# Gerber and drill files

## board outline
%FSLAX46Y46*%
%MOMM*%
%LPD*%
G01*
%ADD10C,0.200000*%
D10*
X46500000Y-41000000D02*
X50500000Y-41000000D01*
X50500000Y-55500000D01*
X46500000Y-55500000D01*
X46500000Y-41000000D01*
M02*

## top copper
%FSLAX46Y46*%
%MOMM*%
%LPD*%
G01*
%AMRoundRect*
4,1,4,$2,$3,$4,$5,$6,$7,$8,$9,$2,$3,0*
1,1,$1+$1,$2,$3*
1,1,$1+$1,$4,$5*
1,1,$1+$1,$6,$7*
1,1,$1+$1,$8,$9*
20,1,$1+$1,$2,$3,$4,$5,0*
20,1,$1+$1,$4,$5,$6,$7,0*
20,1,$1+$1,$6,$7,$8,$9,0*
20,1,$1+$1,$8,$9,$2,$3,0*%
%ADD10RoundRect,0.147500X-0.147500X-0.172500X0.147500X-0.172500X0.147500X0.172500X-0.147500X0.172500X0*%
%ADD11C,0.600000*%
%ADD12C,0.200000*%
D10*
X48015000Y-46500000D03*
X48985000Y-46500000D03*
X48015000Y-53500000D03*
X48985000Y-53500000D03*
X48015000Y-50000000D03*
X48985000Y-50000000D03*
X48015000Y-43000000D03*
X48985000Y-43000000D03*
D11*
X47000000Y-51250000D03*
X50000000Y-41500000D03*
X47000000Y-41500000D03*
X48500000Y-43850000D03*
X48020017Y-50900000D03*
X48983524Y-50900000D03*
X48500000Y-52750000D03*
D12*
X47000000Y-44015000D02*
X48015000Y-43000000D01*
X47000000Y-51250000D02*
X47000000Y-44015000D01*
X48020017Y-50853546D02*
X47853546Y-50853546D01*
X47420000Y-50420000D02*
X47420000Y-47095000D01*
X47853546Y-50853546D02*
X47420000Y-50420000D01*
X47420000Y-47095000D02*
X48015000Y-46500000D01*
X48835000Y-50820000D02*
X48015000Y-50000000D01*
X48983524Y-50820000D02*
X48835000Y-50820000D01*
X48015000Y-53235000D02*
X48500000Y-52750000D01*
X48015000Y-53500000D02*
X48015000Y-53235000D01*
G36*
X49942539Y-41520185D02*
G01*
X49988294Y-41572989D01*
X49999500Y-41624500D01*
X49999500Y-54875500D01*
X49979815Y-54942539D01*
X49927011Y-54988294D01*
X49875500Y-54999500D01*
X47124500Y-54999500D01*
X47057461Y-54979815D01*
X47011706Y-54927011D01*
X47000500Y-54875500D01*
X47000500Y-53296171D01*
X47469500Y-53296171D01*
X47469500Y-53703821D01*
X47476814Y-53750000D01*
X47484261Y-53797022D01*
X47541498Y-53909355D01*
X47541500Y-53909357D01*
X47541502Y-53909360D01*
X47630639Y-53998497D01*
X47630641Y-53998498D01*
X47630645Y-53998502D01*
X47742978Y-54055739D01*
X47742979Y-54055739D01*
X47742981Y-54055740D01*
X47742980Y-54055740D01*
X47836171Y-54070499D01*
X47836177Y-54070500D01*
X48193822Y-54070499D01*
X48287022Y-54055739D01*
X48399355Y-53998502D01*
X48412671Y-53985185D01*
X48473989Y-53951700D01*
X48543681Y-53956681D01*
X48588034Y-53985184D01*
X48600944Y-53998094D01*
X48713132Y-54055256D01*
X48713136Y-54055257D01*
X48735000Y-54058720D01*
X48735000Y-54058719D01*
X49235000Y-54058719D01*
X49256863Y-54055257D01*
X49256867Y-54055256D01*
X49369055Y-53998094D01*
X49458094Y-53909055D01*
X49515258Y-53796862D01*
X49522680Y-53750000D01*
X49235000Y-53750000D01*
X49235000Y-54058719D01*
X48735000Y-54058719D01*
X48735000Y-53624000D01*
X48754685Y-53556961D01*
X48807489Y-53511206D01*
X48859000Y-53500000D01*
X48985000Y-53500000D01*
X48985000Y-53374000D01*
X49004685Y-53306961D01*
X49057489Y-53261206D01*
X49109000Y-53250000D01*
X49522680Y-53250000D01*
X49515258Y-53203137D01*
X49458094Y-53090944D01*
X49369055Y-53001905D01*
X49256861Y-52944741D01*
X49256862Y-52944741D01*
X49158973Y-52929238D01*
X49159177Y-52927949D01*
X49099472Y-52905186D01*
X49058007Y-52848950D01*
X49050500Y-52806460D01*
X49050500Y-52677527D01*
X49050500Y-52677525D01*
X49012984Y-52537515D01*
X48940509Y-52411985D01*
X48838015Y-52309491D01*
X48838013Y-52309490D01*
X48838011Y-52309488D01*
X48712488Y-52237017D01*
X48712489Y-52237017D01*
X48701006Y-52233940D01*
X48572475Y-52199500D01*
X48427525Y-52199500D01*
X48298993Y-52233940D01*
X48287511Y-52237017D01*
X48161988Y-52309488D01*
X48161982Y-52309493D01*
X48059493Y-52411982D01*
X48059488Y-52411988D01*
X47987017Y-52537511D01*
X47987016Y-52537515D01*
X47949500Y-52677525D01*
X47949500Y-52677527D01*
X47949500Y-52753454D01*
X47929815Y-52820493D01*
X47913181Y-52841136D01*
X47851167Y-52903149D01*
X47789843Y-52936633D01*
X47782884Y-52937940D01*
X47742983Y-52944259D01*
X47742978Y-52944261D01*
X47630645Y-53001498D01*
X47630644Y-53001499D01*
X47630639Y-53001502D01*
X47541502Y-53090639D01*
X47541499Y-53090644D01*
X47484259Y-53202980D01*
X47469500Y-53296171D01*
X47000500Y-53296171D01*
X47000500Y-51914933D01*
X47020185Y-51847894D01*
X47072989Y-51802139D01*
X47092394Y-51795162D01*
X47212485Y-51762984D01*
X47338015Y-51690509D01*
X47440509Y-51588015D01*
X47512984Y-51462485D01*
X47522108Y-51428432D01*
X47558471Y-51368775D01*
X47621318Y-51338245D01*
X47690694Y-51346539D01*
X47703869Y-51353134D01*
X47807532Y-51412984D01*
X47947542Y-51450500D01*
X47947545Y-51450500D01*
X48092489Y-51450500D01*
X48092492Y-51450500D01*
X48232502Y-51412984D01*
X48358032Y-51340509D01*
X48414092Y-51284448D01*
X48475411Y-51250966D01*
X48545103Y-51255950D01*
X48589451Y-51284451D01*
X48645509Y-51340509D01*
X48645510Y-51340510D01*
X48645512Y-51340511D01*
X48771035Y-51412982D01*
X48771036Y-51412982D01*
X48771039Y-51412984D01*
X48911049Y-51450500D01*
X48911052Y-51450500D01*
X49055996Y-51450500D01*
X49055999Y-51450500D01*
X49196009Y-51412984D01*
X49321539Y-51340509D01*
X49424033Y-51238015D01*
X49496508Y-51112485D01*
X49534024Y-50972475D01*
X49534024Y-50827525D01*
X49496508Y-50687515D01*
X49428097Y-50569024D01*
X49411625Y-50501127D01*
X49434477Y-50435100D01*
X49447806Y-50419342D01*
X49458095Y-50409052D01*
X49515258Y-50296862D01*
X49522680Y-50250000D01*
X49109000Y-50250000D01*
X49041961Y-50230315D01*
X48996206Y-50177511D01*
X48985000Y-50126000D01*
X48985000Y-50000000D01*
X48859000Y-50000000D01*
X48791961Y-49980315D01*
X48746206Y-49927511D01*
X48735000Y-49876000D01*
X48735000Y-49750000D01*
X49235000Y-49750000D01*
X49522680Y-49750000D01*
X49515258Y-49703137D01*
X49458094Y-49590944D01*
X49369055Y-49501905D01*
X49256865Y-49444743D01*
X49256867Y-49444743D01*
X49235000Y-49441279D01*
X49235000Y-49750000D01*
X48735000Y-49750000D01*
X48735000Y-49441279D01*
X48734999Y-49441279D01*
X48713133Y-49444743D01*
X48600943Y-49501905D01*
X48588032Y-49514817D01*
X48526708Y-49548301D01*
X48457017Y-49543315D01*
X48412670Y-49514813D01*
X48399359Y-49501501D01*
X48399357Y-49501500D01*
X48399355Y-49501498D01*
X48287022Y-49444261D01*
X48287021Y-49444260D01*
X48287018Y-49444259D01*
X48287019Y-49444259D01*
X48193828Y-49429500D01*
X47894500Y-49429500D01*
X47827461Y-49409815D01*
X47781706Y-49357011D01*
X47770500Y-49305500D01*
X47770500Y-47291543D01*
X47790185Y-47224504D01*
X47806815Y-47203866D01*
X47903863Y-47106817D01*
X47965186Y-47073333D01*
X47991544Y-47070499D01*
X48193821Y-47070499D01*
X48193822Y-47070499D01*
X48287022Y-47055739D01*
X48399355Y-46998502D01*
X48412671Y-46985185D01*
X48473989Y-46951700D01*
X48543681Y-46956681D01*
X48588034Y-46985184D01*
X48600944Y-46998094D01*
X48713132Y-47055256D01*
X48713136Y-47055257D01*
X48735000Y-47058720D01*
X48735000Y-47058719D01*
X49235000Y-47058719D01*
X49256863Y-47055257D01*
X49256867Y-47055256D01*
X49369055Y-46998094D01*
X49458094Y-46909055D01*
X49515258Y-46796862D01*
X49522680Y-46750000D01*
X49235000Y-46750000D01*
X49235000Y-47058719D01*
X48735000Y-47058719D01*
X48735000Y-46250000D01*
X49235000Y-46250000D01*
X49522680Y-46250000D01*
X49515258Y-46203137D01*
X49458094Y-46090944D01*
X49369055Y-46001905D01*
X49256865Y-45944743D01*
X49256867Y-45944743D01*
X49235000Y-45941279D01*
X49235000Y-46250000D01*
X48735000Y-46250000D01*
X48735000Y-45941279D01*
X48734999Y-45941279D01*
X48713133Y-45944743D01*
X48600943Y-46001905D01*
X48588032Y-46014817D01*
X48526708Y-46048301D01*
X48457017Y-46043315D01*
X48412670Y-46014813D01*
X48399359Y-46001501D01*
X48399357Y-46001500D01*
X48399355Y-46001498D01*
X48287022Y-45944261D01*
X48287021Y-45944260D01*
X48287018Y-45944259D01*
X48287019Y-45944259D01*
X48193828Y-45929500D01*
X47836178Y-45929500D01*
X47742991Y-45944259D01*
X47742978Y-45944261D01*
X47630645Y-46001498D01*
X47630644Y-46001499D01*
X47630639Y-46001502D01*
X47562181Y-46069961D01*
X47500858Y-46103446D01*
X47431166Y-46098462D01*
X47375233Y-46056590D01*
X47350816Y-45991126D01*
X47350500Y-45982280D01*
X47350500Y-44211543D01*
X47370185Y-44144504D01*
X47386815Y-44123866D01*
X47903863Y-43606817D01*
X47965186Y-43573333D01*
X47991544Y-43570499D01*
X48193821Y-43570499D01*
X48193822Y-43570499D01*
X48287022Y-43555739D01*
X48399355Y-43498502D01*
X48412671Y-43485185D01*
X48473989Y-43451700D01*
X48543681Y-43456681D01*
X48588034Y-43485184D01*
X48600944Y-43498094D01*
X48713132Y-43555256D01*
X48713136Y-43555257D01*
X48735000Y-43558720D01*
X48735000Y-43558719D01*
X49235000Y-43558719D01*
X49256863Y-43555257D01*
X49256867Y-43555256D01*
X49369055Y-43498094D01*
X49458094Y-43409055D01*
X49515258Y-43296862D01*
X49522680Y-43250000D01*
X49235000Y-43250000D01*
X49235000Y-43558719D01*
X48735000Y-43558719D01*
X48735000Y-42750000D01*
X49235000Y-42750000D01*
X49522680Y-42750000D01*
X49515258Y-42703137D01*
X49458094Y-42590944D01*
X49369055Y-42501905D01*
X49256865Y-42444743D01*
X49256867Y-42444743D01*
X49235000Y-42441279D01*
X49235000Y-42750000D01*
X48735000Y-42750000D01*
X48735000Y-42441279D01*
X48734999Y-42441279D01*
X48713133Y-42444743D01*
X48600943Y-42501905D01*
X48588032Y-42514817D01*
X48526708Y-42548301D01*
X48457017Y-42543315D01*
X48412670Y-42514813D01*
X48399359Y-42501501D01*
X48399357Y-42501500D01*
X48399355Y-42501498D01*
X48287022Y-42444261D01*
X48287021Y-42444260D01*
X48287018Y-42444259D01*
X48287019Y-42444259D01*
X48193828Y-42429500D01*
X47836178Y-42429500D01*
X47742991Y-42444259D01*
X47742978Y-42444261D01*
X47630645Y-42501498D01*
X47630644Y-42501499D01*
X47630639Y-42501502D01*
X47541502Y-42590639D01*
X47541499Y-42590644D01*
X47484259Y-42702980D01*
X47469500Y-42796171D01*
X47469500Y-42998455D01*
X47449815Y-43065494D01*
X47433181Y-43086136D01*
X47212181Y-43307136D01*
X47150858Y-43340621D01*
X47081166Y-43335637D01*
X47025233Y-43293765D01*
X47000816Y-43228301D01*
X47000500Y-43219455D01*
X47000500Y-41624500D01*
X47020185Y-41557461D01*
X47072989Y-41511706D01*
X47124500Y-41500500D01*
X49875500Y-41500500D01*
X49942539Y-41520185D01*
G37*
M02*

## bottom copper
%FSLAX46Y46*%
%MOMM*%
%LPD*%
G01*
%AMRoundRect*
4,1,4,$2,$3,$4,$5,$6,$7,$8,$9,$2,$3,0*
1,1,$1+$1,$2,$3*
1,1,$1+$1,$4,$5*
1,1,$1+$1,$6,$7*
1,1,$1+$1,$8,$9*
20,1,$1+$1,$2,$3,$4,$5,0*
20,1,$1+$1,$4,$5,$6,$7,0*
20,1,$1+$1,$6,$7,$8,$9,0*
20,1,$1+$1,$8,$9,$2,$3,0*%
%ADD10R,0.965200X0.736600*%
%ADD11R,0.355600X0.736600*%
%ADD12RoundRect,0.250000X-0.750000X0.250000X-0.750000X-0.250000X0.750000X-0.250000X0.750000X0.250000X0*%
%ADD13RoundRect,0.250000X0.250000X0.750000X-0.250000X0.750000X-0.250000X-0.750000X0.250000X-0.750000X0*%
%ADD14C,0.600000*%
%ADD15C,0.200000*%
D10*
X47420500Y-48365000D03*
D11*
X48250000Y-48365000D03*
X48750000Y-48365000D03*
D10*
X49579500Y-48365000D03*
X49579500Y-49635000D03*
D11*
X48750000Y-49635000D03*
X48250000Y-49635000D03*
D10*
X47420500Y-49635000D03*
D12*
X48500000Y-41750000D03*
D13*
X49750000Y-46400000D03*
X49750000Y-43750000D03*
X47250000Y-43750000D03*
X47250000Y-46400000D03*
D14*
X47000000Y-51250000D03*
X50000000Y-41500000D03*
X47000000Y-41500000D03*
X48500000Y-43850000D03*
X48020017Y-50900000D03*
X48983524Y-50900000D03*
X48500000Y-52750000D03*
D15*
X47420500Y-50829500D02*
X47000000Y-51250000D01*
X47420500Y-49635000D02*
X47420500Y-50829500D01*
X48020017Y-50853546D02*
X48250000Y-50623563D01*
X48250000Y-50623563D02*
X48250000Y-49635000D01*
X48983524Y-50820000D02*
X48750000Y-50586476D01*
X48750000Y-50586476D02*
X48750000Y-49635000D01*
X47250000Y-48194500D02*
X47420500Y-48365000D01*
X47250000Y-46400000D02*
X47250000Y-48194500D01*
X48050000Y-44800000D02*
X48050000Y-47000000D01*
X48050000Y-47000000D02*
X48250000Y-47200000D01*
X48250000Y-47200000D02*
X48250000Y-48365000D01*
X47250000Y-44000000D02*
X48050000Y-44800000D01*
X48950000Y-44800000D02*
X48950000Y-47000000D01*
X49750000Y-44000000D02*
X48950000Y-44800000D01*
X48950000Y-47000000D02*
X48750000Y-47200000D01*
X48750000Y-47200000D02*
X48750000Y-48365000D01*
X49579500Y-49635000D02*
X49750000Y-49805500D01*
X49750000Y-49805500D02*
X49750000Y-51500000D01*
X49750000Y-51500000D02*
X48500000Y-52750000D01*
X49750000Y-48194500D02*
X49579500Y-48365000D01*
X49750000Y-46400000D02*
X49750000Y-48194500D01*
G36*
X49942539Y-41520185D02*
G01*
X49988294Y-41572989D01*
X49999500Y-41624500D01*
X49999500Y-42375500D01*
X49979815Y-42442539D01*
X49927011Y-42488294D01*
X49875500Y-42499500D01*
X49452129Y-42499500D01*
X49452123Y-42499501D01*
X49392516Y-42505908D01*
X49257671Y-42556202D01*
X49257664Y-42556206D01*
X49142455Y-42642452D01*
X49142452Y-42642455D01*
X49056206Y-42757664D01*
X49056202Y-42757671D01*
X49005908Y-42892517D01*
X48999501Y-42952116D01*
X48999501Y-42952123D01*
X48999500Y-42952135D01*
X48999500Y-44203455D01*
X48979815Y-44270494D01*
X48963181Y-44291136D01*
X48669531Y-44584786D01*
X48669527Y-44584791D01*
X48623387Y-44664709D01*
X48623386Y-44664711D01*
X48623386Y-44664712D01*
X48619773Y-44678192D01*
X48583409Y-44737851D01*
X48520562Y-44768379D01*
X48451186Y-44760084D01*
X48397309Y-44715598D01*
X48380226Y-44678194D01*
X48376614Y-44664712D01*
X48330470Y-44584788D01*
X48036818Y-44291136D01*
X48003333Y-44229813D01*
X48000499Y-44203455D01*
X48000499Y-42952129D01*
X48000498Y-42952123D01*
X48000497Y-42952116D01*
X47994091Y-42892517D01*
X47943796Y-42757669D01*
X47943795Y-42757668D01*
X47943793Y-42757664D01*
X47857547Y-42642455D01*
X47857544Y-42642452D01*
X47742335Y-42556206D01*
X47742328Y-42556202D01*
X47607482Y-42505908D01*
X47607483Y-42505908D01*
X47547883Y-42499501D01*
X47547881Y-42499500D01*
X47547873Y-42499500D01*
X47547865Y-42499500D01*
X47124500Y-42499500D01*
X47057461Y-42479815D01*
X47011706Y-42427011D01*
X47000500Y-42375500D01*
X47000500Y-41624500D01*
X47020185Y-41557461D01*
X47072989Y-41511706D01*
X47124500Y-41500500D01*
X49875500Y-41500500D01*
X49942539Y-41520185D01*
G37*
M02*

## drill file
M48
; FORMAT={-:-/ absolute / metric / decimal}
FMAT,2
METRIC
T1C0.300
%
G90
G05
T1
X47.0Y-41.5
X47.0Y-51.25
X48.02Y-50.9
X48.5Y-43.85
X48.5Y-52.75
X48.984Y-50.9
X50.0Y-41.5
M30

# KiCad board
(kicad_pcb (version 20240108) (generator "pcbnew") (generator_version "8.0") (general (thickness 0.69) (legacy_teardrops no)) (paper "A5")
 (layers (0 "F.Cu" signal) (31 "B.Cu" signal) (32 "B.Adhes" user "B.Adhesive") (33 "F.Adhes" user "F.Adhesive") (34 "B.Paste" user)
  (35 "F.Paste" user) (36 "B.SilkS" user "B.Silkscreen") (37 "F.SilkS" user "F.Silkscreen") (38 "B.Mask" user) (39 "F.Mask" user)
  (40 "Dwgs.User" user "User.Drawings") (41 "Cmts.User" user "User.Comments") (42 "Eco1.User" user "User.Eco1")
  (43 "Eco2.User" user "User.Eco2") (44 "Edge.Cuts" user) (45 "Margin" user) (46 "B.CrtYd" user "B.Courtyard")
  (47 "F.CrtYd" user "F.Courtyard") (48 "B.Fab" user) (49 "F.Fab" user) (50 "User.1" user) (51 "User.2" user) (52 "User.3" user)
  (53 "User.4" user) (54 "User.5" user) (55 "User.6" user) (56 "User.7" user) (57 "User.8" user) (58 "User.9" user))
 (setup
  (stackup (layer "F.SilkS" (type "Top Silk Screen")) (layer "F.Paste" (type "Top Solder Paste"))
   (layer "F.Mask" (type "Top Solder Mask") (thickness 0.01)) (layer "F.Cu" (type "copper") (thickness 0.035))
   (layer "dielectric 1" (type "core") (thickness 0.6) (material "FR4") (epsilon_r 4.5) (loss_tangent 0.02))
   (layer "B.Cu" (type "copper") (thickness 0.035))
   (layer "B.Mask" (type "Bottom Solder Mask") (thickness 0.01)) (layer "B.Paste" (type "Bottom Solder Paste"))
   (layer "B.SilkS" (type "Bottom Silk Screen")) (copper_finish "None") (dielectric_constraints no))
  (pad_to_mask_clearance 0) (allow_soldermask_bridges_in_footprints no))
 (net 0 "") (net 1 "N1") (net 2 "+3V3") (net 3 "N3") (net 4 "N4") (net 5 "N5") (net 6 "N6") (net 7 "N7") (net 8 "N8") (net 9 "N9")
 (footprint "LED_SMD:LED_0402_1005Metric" (layer "F.Cu") (at 48.5 46.5)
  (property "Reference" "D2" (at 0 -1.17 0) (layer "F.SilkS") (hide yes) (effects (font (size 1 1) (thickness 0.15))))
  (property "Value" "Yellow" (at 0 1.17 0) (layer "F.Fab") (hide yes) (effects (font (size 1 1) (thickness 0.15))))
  (pad "1" smd roundrect (at -0.485 0) (size 0.59 0.64) (layers "F.Cu" "F.Paste" "F.Mask") (roundrect_rratio 0.25) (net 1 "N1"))
  (pad "2" smd roundrect (at 0.485 0) (size 0.59 0.64) (layers "F.Cu" "F.Paste" "F.Mask") (roundrect_rratio 0.25) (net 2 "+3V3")))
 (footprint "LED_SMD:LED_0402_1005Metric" (layer "F.Cu") (at 48.5 53.5)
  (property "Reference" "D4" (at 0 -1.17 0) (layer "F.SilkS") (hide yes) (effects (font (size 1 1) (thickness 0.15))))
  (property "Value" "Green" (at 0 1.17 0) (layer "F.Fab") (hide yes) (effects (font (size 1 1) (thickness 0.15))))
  (pad "1" smd roundrect (at -0.485 0) (size 0.59 0.64) (layers "F.Cu" "F.Paste" "F.Mask") (roundrect_rratio 0.25) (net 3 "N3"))
  (pad "2" smd roundrect (at 0.485 0) (size 0.59 0.64) (layers "F.Cu" "F.Paste" "F.Mask") (roundrect_rratio 0.25) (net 2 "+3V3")))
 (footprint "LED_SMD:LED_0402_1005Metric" (layer "F.Cu") (at 48.5 50)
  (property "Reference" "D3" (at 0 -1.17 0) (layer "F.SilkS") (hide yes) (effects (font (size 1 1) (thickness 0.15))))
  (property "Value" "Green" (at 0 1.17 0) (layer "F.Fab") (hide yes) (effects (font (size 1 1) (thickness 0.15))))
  (pad "1" smd roundrect (at -0.485 0) (size 0.59 0.64) (layers "F.Cu" "F.Paste" "F.Mask") (roundrect_rratio 0.25) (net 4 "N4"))
  (pad "2" smd roundrect (at 0.485 0) (size 0.59 0.64) (layers "F.Cu" "F.Paste" "F.Mask") (roundrect_rratio 0.25) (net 2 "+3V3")))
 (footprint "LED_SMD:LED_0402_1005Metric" (layer "F.Cu") (at 48.5 43)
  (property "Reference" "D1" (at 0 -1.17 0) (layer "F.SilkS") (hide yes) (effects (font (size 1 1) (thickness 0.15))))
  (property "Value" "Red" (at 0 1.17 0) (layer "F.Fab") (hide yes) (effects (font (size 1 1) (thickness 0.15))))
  (pad "1" smd roundrect (at -0.485 0) (size 0.59 0.64) (layers "F.Cu" "F.Paste" "F.Mask") (roundrect_rratio 0.25) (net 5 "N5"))
  (pad "2" smd roundrect (at 0.485 0) (size 0.59 0.64) (layers "F.Cu" "F.Paste" "F.Mask") (roundrect_rratio 0.25) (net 2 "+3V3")))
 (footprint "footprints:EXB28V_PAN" (layer "B.Cu") (at 48.5 49 -90)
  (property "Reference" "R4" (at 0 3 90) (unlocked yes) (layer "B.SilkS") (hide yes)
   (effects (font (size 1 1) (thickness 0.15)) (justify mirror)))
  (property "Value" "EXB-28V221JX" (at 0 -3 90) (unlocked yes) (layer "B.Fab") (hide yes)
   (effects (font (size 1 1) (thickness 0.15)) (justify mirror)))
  (pad "1" smd rect (at -0.635 1.0795 270) (size 0.7366 0.9652) (layers "B.Cu" "B.Paste" "B.Mask") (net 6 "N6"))
  (pad "2" smd rect (at -0.635 0.25 270) (size 0.7366 0.3556) (layers "B.Cu" "B.Paste" "B.Mask") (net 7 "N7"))
  (pad "3" smd rect (at -0.635 -0.25 270) (size 0.7366 0.3556) (layers "B.Cu" "B.Paste" "B.Mask") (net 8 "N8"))
  (pad "4" smd rect (at -0.635 -1.0795 270) (size 0.7366 0.9652) (layers "B.Cu" "B.Paste" "B.Mask") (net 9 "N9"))
  (pad "5" smd rect (at 0.635 -1.0795 270) (size 0.7366 0.9652) (layers "B.Cu" "B.Paste" "B.Mask") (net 3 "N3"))
  (pad "6" smd rect (at 0.635 -0.25 270) (size 0.7366 0.3556) (layers "B.Cu" "B.Paste" "B.Mask") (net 4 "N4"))
  (pad "7" smd rect (at 0.635 0.25 270) (size 0.7366 0.3556) (layers "B.Cu" "B.Paste" "B.Mask") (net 1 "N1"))
  (pad "8" smd rect (at 0.635 1.0795 270) (size 0.7366 0.9652) (layers "B.Cu" "B.Paste" "B.Mask") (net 5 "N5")))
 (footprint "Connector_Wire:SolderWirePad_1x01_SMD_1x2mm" (layer "B.Cu") (at 48.5 41.75 -90)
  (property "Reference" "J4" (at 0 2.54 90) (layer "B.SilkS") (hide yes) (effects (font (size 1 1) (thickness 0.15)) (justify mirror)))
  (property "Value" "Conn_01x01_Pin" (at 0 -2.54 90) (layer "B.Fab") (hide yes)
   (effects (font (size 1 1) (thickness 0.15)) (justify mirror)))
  (pad "1" smd roundrect (at 0 0 270) (size 1 2) (layers "B.Cu" "B.Paste" "B.Mask") (roundrect_rratio 0.25) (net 2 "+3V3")))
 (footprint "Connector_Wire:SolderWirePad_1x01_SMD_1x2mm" (layer "B.Cu") (at 49.75 46.4 180)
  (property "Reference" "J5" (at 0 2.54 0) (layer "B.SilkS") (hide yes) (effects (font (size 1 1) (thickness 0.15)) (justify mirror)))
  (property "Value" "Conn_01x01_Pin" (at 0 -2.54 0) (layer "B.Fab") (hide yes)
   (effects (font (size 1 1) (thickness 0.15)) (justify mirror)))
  (pad "1" smd roundrect (at 0 0 180) (size 1 2) (layers "B.Cu" "B.Paste" "B.Mask") (roundrect_rratio 0.25) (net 9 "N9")))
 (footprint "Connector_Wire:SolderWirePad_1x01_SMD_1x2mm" (layer "B.Cu") (at 49.75 43.75 180)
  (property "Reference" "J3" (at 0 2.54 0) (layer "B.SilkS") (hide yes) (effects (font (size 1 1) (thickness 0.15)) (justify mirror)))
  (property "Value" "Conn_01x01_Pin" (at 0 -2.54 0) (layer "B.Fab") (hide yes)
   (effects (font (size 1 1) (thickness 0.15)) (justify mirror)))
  (pad "1" smd roundrect (at 0 0 180) (size 1 2) (layers "B.Cu" "B.Paste" "B.Mask") (roundrect_rratio 0.25) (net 8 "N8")))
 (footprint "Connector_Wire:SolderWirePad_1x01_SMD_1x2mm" (layer "B.Cu") (at 47.25 43.75 180)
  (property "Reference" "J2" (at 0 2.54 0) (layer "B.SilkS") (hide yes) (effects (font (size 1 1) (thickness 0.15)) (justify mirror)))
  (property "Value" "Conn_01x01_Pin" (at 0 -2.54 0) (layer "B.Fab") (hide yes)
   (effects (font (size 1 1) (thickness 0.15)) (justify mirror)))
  (pad "1" smd roundrect (at 0 0 180) (size 1 2) (layers "B.Cu" "B.Paste" "B.Mask") (roundrect_rratio 0.25) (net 7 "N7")))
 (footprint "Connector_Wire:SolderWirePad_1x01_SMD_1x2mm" (layer "B.Cu") (at 47.25 46.4 180)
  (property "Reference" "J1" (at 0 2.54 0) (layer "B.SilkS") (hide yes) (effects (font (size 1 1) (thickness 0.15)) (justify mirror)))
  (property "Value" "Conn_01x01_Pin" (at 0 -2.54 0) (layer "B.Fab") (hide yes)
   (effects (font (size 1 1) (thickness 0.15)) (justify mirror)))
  (pad "1" smd roundrect (at 0 0 180) (size 1 2) (layers "B.Cu" "B.Paste" "B.Mask") (roundrect_rratio 0.25) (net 6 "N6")))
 (gr_rect (start 46.5 41) (end 50.5 55.5) (stroke (width 0.2) (type default)) (fill none) (layer "Edge.Cuts"))
 (segment (start 47 44.015) (end 48.015 43) (width 0.2) (layer "F.Cu") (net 5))
 (segment (start 47 51.25) (end 47 44.015) (width 0.2) (layer "F.Cu") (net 5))
 (via (at 47 51.25) (size 0.6) (drill 0.3) (layers "F.Cu" "B.Cu") (free yes) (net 5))
 (segment (start 47.4205 50.8295) (end 47 51.25) (width 0.2) (layer "B.Cu") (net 5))
 (segment (start 47.4205 49.635) (end 47.4205 50.8295) (width 0.2) (layer "B.Cu") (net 5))
 (via (at 50 41.5) (size 0.6) (drill 0.3) (layers "F.Cu" "B.Cu") (free yes) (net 2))
 (via (at 47 41.5) (size 0.6) (drill 0.3) (layers "F.Cu" "B.Cu") (free yes) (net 2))
 (via (at 48.5 43.85) (size 0.6) (drill 0.3) (layers "F.Cu" "B.Cu") (free yes) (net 2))
 (segment (start 48.020017 50.853546) (end 47.853546 50.853546) (width 0.2) (layer "F.Cu") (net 1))
 (segment (start 47.42 50.42) (end 47.42 47.095) (width 0.2) (layer "F.Cu") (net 1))
 (segment (start 47.853546 50.853546) (end 47.42 50.42) (width 0.2) (layer "F.Cu") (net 1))
 (segment (start 47.42 47.095) (end 48.015 46.5) (width 0.2) (layer "F.Cu") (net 1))
 (via (at 48.020017 50.9) (size 0.6) (drill 0.3) (layers "F.Cu" "B.Cu") (free yes) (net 1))
 (segment (start 48.020017 50.853546) (end 48.25 50.623563) (width 0.2) (layer "B.Cu") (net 1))
 (segment (start 48.25 50.623563) (end 48.25 49.635) (width 0.2) (layer "B.Cu") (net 1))
 (segment (start 48.835 50.82) (end 48.015 50) (width 0.2) (layer "F.Cu") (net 4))
 (segment (start 48.983524 50.82) (end 48.835 50.82) (width 0.2) (layer "F.Cu") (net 4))
 (via (at 48.983524 50.9) (size 0.6) (drill 0.3) (layers "F.Cu" "B.Cu") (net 4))
 (segment (start 48.983524 50.82) (end 48.75 50.586476) (width 0.2) (layer "B.Cu") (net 4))
 (segment (start 48.75 50.586476) (end 48.75 49.635) (width 0.2) (layer "B.Cu") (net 4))
 (segment (start 47.25 48.1945) (end 47.4205 48.365) (width 0.2) (layer "B.Cu") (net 6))
 (segment (start 47.25 46.4) (end 47.25 48.1945) (width 0.2) (layer "B.Cu") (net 6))
 (segment (start 48.05 44.8) (end 48.05 47) (width 0.2) (layer "B.Cu") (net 7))
 (segment (start 48.05 47) (end 48.25 47.2) (width 0.2) (layer "B.Cu") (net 7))
 (segment (start 48.25 47.2) (end 48.25 48.365) (width 0.2) (layer "B.Cu") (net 7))
 (segment (start 47.25 44) (end 48.05 44.8) (width 0.2) (layer "B.Cu") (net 7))
 (segment (start 48.95 44.8) (end 48.95 47) (width 0.2) (layer "B.Cu") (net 8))
 (segment (start 49.75 44) (end 48.95 44.8) (width 0.2) (layer "B.Cu") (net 8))
 (segment (start 48.95 47) (end 48.75 47.2) (width 0.2) (layer "B.Cu") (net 8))
 (segment (start 48.75 47.2) (end 48.75 48.365) (width 0.2) (layer "B.Cu") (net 8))
 (segment (start 48.015 53.235) (end 48.5 52.75) (width 0.2) (layer "F.Cu") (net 3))
 (segment (start 48.015 53.5) (end 48.015 53.235) (width 0.2) (layer "F.Cu") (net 3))
 (via (at 48.5 52.75) (size 0.6) (drill 0.3) (layers "F.Cu" "B.Cu") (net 3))
 (segment (start 49.5795 49.635) (end 49.75 49.8055) (width 0.2) (layer "B.Cu") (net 3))
 (segment (start 49.75 49.8055) (end 49.75 51.5) (width 0.2) (layer "B.Cu") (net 3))
 (segment (start 49.75 51.5) (end 48.5 52.75) (width 0.2) (layer "B.Cu") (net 3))
 (segment (start 49.75 48.1945) (end 49.5795 48.365) (width 0.2) (layer "B.Cu") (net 9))
 (segment (start 49.75 46.4) (end 49.75 48.1945) (width 0.2) (layer "B.Cu") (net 9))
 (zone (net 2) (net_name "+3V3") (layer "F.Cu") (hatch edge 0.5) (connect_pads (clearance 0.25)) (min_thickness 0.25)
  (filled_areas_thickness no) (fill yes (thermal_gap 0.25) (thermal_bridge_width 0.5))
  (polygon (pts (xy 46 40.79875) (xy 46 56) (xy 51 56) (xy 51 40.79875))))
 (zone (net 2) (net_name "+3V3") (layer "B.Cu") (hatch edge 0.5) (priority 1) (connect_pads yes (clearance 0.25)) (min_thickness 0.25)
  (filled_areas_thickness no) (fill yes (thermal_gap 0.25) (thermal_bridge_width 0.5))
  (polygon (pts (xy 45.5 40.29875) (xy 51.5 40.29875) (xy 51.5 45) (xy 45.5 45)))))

